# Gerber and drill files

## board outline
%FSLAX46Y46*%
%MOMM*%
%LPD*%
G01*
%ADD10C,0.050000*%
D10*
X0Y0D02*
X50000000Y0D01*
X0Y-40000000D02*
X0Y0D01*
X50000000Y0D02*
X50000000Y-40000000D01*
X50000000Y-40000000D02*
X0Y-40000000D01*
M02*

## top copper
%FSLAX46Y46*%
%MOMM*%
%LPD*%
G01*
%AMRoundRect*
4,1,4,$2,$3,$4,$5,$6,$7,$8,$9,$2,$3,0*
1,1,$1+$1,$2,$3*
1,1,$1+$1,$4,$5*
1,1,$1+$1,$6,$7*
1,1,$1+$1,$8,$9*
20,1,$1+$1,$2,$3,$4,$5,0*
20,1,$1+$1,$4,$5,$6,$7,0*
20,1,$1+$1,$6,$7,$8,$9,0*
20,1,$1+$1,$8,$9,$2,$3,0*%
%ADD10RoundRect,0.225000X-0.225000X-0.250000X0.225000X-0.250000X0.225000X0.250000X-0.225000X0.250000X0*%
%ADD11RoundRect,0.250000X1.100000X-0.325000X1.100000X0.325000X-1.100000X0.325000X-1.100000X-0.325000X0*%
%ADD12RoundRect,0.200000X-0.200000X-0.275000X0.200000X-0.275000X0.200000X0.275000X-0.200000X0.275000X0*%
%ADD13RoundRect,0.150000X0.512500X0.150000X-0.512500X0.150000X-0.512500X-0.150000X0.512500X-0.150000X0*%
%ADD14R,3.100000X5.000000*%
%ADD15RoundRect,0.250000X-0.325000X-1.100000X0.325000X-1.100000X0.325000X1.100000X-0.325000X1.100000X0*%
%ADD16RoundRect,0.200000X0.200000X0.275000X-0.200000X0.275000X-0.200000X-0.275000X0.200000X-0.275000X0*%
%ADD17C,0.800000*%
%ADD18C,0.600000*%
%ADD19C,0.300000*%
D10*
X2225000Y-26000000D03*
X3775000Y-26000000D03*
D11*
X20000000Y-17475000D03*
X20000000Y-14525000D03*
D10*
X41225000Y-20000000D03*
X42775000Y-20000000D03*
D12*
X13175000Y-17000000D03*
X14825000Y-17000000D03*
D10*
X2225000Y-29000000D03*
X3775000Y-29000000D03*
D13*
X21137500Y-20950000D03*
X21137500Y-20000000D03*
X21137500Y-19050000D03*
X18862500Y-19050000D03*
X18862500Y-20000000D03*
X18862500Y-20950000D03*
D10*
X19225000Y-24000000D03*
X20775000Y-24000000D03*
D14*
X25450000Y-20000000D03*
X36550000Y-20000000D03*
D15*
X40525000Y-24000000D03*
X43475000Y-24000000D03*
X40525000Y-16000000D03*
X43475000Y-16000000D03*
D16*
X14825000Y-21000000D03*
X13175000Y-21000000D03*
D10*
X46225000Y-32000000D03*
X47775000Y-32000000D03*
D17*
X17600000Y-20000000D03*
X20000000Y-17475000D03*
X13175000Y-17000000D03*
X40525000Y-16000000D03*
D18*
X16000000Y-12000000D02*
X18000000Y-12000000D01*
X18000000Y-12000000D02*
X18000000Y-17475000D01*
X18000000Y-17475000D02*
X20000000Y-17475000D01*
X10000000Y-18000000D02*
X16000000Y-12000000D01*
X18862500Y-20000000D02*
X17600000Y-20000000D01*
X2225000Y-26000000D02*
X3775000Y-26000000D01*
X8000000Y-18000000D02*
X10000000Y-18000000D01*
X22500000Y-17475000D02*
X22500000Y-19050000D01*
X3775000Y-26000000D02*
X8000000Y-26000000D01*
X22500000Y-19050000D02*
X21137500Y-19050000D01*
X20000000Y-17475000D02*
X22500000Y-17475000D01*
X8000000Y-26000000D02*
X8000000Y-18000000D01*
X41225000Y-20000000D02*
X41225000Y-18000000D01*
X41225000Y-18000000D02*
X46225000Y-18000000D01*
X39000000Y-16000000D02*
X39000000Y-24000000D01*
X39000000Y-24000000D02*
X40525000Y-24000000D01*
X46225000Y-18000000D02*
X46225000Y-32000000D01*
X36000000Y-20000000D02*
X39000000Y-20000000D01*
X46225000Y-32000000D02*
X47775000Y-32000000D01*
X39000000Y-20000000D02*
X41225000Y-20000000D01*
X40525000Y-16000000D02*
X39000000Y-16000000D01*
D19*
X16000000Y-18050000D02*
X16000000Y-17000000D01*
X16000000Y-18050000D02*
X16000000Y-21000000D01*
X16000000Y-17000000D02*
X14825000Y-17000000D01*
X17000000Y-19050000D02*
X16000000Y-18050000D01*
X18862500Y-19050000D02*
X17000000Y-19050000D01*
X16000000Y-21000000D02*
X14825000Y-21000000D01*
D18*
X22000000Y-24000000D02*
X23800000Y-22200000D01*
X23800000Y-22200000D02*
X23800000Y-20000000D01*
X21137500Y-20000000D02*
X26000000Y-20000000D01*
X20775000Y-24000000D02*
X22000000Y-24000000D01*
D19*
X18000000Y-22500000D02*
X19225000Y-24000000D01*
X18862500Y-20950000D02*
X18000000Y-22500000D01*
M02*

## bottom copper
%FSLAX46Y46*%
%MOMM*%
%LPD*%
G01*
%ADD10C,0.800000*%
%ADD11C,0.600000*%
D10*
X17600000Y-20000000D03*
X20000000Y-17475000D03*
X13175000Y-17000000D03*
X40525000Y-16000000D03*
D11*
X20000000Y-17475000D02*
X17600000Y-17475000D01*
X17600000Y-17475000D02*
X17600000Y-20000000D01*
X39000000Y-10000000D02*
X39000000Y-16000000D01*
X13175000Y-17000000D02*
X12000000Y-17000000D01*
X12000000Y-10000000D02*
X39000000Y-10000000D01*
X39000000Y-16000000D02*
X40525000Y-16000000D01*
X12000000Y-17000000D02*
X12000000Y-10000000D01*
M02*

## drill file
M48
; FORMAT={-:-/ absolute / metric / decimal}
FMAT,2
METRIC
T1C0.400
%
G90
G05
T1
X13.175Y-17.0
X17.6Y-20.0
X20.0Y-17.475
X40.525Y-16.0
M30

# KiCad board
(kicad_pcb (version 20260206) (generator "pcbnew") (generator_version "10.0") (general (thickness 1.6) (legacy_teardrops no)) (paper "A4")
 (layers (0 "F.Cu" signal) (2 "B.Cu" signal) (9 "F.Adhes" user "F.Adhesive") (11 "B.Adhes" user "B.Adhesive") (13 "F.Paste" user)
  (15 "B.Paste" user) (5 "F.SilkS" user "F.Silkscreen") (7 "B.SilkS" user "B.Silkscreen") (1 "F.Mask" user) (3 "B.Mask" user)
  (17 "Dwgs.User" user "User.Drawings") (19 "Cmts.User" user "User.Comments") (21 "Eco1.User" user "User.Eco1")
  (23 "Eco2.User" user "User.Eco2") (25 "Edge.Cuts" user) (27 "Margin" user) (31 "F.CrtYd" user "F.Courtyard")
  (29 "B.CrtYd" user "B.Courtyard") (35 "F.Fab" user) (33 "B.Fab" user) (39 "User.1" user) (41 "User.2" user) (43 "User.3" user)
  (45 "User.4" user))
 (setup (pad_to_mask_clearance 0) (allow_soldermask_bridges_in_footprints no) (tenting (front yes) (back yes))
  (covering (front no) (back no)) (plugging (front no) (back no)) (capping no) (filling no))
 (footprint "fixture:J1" (layer "F.Cu") (at 3 26)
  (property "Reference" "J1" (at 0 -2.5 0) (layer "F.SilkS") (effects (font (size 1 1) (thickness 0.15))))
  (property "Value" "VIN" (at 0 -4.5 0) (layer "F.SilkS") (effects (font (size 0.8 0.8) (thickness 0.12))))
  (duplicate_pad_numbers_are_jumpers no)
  (pad "1" smd roundrect (at -0.775 0) (size 0.9 0.95) (layers "F.Cu" "F.Mask" "F.Paste") (roundrect_rratio 0.25) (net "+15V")
   (thermal_bridge_angle 45))
  (pad "2" smd roundrect (at 0.775 0) (size 0.9 0.95) (layers "F.Cu" "F.Mask" "F.Paste") (roundrect_rratio 0.25) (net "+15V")
   (thermal_bridge_angle 45)))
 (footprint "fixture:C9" (layer "F.Cu") (at 20 16 90)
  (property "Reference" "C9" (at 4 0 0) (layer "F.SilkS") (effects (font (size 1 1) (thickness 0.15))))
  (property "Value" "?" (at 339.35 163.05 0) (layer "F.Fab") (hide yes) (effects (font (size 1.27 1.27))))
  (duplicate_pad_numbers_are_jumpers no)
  (pad "1" smd roundrect (at -1.475 0 90) (size 1.15 2.7) (layers "F.Cu" "F.Mask" "F.Paste") (roundrect_rratio 0.217391) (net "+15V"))
  (pad "2" smd roundrect (at 1.475 0 90) (size 1.15 2.7) (layers "F.Cu" "F.Mask" "F.Paste") (roundrect_rratio 0.217391) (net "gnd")))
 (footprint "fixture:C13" (layer "F.Cu") (at 42 20)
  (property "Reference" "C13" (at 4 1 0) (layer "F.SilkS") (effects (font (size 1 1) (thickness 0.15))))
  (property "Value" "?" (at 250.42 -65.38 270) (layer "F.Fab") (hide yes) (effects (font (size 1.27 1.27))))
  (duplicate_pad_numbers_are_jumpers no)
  (pad "1" smd roundrect (at -0.775 0) (size 0.9 0.95) (layers "F.Cu" "F.Mask" "F.Paste") (roundrect_rratio 0.25) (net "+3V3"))
  (pad "2" smd roundrect (at 0.775 0) (size 0.9 0.95) (layers "F.Cu" "F.Mask" "F.Paste") (roundrect_rratio 0.25) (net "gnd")))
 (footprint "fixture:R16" (layer "F.Cu") (at 14 17)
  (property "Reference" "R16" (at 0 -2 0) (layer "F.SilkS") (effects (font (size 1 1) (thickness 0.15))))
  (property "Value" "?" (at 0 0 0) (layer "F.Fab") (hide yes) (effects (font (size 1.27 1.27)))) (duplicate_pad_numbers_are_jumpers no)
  (pad "1" smd roundrect (at -0.825 0) (size 0.8 0.95) (layers "F.Cu" "F.Mask" "F.Paste") (roundrect_rratio 0.25) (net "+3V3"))
  (pad "2" smd roundrect (at 0.825 0) (size 0.8 0.95) (layers "F.Cu" "F.Mask" "F.Paste") (roundrect_rratio 0.25) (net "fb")))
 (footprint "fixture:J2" (layer "F.Cu") (at 3 29)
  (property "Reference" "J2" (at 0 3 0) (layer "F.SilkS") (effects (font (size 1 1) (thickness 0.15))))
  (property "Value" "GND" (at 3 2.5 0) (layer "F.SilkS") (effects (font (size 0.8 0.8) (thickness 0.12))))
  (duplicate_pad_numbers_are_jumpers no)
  (pad "1" smd roundrect (at -0.775 0) (size 0.9 0.95) (layers "F.Cu" "F.Mask" "F.Paste") (roundrect_rratio 0.25) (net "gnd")
   (thermal_bridge_angle 45))
  (pad "2" smd roundrect (at 0.775 0) (size 0.9 0.95) (layers "F.Cu" "F.Mask" "F.Paste") (roundrect_rratio 0.25) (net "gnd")
   (thermal_bridge_angle 45)))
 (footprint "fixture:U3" (layer "F.Cu") (at 20 20 180)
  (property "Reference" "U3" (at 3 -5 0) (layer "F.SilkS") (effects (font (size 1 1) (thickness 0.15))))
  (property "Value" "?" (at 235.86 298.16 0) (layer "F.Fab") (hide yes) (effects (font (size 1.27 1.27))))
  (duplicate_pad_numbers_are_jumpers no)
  (pad "1" smd roundrect (at -1.1375 -0.95 180) (size 1.325 0.6) (layers "F.Cu" "F.Mask" "F.Paste") (roundrect_rratio 0.25) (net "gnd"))
  (pad "2" smd roundrect (at -1.1375 0 180) (size 1.325 0.6) (layers "F.Cu" "F.Mask" "F.Paste") (roundrect_rratio 0.25) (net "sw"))
  (pad "3" smd roundrect (at -1.1375 0.95 180) (size 1.325 0.6) (layers "F.Cu" "F.Mask" "F.Paste") (roundrect_rratio 0.25) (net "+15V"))
  (pad "4" smd roundrect (at 1.1375 0.95 180) (size 1.325 0.6) (layers "F.Cu" "F.Mask" "F.Paste") (roundrect_rratio 0.25) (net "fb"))
  (pad "5" smd roundrect (at 1.1375 0 180) (size 1.325 0.6) (layers "F.Cu" "F.Mask" "F.Paste") (roundrect_rratio 0.25) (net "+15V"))
  (pad "6" smd roundrect (at 1.1375 -0.95 180) (size 1.325 0.6) (layers "F.Cu" "F.Mask" "F.Paste") (roundrect_rratio 0.25) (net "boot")))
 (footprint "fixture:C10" (layer "F.Cu") (at 20 24)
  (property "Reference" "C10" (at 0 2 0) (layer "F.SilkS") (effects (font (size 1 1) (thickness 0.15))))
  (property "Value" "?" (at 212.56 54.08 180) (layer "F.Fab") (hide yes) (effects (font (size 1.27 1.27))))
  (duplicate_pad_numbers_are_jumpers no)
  (pad "1" smd roundrect (at -0.775 0) (size 0.9 0.95) (layers "F.Cu" "F.Mask" "F.Paste") (roundrect_rratio 0.25) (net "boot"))
  (pad "2" smd roundrect (at 0.775 0) (size 0.9 0.95) (layers "F.Cu" "F.Mask" "F.Paste") (roundrect_rratio 0.25) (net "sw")))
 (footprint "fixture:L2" (layer "F.Cu") (at 31 20)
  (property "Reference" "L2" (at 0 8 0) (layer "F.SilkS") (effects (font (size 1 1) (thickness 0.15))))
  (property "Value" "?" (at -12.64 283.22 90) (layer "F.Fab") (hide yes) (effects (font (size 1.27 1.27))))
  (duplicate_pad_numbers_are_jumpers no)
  (pad "1" smd rect (at -5.55 0) (size 3.1 5) (layers "F.Cu" "F.Mask" "F.Paste") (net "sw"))
  (pad "2" smd rect (at 5.55 0) (size 3.1 5) (layers "F.Cu" "F.Mask" "F.Paste") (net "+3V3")))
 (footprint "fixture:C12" (layer "F.Cu") (at 42 24)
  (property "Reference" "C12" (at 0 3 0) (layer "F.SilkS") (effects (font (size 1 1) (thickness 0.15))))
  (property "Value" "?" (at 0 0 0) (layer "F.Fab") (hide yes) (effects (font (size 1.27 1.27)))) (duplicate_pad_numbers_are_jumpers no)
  (pad "1" smd roundrect (at -1.475 0) (size 1.15 2.7) (layers "F.Cu" "F.Mask" "F.Paste") (roundrect_rratio 0.217391) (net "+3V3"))
  (pad "2" smd roundrect (at 1.475 0) (size 1.15 2.7) (layers "F.Cu" "F.Mask" "F.Paste") (roundrect_rratio 0.217391) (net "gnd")))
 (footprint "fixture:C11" (layer "F.Cu") (at 42 16)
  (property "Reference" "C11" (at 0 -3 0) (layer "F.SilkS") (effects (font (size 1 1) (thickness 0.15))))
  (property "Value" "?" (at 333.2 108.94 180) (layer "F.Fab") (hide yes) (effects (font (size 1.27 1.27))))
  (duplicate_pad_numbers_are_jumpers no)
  (pad "1" smd roundrect (at -1.475 0) (size 1.15 2.7) (layers "F.Cu" "F.Mask" "F.Paste") (roundrect_rratio 0.217391) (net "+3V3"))
  (pad "2" smd roundrect (at 1.475 0) (size 1.15 2.7) (layers "F.Cu" "F.Mask" "F.Paste") (roundrect_rratio 0.217391) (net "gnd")))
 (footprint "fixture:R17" (layer "F.Cu") (at 14 21 180)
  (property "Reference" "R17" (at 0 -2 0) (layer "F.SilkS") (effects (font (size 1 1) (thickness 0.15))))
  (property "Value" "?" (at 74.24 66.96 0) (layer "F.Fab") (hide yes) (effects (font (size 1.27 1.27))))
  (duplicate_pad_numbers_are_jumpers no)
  (pad "1" smd roundrect (at -0.825 0 180) (size 0.8 0.95) (layers "F.Cu" "F.Mask" "F.Paste") (roundrect_rratio 0.25) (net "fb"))
  (pad "2" smd roundrect (at 0.825 0 180) (size 0.8 0.95) (layers "F.Cu" "F.Mask" "F.Paste") (roundrect_rratio 0.25) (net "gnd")))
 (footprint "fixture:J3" (layer "F.Cu") (at 47 32)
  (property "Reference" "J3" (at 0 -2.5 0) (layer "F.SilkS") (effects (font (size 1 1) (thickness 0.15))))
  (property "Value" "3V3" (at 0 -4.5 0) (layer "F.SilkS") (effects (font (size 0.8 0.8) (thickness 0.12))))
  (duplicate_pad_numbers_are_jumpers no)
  (pad "1" smd roundrect (at -0.775 0) (size 0.9 0.95) (layers "F.Cu" "F.Mask" "F.Paste") (roundrect_rratio 0.25) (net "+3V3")
   (thermal_bridge_angle 45))
  (pad "2" smd roundrect (at 0.775 0) (size 0.9 0.95) (layers "F.Cu" "F.Mask" "F.Paste") (roundrect_rratio 0.25) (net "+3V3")
   (thermal_bridge_angle 45)))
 (gr_line (start 0 0) (end 50 0) (stroke (width 0.05) (type default)) (layer "Edge.Cuts"))
 (gr_line (start 0 40) (end 0 0) (stroke (width 0.05) (type default)) (layer "Edge.Cuts"))
 (gr_line (start 50 0) (end 50 40) (stroke (width 0.05) (type default)) (layer "Edge.Cuts"))
 (gr_line (start 50 40) (end 0 40) (stroke (width 0.05) (type default)) (layer "Edge.Cuts"))
 (segment (start 16 12) (end 18 12) (width 0.6) (layer "F.Cu") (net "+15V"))
 (segment (start 18 12) (end 18 17.475) (width 0.6) (layer "F.Cu") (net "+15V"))
 (segment (start 18 17.475) (end 20 17.475) (width 0.6) (layer "F.Cu") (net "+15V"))
 (segment (start 10 18) (end 16 12) (width 0.6) (layer "F.Cu") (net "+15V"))
 (segment (start 18.8625 20) (end 17.6 20) (width 0.6) (layer "F.Cu") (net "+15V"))
 (segment (start 2.225 26) (end 3.775 26) (width 0.6) (layer "F.Cu") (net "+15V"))
 (segment (start 8 18) (end 10 18) (width 0.6) (layer "F.Cu") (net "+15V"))
 (segment (start 22.5 17.475) (end 22.5 19.05) (width 0.6) (layer "F.Cu") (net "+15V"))
 (segment (start 3.775 26) (end 8 26) (width 0.6) (layer "F.Cu") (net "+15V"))
 (segment (start 22.5 19.05) (end 21.1375 19.05) (width 0.6) (layer "F.Cu") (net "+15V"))
 (segment (start 20 17.475) (end 22.5 17.475) (width 0.6) (layer "F.Cu") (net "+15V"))
 (segment (start 8 26) (end 8 18) (width 0.6) (layer "F.Cu") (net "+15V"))
 (via (at 17.6 20) (size 0.8) (drill 0.4) (layers "F.Cu" "B.Cu") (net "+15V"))
 (via (at 20 17.475) (size 0.8) (drill 0.4) (layers "F.Cu" "B.Cu") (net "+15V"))
 (segment (start 20 17.475) (end 17.6 17.475) (width 0.6) (layer "B.Cu") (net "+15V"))
 (segment (start 17.6 17.475) (end 17.6 20) (width 0.6) (layer "B.Cu") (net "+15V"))
 (segment (start 41.225 20) (end 41.225 18) (width 0.6) (layer "F.Cu") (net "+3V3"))
 (segment (start 41.225 18) (end 46.225 18) (width 0.6) (layer "F.Cu") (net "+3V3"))
 (segment (start 39 16) (end 39 24) (width 0.6) (layer "F.Cu") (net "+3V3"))
 (segment (start 39 24) (end 40.525 24) (width 0.6) (layer "F.Cu") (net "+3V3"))
 (segment (start 46.225 18) (end 46.225 32) (width 0.6) (layer "F.Cu") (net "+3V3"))
 (segment (start 36 20) (end 39 20) (width 0.6) (layer "F.Cu") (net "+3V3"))
 (segment (start 46.225 32) (end 47.775 32) (width 0.6) (layer "F.Cu") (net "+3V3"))
 (segment (start 39 20) (end 41.225 20) (width 0.6) (layer "F.Cu") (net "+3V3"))
 (segment (start 40.525 16) (end 39 16) (width 0.6) (layer "F.Cu") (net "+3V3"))
 (via (at 13.175 17) (size 0.8) (drill 0.4) (layers "F.Cu" "B.Cu") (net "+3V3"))
 (via (at 40.525 16) (size 0.8) (drill 0.4) (layers "F.Cu" "B.Cu") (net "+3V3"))
 (segment (start 39 10) (end 39 16) (width 0.6) (layer "B.Cu") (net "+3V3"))
 (segment (start 13.175 17) (end 12 17) (width 0.6) (layer "B.Cu") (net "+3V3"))
 (segment (start 12 10) (end 39 10) (width 0.6) (layer "B.Cu") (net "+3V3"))
 (segment (start 39 16) (end 40.525 16) (width 0.6) (layer "B.Cu") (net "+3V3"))
 (segment (start 12 17) (end 12 10) (width 0.6) (layer "B.Cu") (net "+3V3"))
 (segment (start 16 18.05) (end 16 17) (width 0.3) (layer "F.Cu") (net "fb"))
 (segment (start 16 18.05) (end 16 21) (width 0.3) (layer "F.Cu") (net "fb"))
 (segment (start 16 17) (end 14.825 17) (width 0.3) (layer "F.Cu") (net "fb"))
 (segment (start 17 19.05) (end 16 18.05) (width 0.3) (layer "F.Cu") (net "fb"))
 (segment (start 18.8625 19.05) (end 17 19.05) (width 0.3) (layer "F.Cu") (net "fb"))
 (segment (start 16 21) (end 14.825 21) (width 0.3) (layer "F.Cu") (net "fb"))
 (segment (start 22 24) (end 23.8 22.2) (width 0.6) (layer "F.Cu") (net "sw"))
 (segment (start 23.8 22.2) (end 23.8 20) (width 0.6) (layer "F.Cu") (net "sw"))
 (segment (start 21.1375 20) (end 26 20) (width 0.6) (layer "F.Cu") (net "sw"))
 (segment (start 20.775 24) (end 22 24) (width 0.6) (layer "F.Cu") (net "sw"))
 (segment (start 18 22.5) (end 19.225 24) (width 0.3) (layer "F.Cu") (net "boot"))
 (segment (start 18.8625 20.95) (end 18 22.5) (width 0.3) (layer "F.Cu") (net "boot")))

